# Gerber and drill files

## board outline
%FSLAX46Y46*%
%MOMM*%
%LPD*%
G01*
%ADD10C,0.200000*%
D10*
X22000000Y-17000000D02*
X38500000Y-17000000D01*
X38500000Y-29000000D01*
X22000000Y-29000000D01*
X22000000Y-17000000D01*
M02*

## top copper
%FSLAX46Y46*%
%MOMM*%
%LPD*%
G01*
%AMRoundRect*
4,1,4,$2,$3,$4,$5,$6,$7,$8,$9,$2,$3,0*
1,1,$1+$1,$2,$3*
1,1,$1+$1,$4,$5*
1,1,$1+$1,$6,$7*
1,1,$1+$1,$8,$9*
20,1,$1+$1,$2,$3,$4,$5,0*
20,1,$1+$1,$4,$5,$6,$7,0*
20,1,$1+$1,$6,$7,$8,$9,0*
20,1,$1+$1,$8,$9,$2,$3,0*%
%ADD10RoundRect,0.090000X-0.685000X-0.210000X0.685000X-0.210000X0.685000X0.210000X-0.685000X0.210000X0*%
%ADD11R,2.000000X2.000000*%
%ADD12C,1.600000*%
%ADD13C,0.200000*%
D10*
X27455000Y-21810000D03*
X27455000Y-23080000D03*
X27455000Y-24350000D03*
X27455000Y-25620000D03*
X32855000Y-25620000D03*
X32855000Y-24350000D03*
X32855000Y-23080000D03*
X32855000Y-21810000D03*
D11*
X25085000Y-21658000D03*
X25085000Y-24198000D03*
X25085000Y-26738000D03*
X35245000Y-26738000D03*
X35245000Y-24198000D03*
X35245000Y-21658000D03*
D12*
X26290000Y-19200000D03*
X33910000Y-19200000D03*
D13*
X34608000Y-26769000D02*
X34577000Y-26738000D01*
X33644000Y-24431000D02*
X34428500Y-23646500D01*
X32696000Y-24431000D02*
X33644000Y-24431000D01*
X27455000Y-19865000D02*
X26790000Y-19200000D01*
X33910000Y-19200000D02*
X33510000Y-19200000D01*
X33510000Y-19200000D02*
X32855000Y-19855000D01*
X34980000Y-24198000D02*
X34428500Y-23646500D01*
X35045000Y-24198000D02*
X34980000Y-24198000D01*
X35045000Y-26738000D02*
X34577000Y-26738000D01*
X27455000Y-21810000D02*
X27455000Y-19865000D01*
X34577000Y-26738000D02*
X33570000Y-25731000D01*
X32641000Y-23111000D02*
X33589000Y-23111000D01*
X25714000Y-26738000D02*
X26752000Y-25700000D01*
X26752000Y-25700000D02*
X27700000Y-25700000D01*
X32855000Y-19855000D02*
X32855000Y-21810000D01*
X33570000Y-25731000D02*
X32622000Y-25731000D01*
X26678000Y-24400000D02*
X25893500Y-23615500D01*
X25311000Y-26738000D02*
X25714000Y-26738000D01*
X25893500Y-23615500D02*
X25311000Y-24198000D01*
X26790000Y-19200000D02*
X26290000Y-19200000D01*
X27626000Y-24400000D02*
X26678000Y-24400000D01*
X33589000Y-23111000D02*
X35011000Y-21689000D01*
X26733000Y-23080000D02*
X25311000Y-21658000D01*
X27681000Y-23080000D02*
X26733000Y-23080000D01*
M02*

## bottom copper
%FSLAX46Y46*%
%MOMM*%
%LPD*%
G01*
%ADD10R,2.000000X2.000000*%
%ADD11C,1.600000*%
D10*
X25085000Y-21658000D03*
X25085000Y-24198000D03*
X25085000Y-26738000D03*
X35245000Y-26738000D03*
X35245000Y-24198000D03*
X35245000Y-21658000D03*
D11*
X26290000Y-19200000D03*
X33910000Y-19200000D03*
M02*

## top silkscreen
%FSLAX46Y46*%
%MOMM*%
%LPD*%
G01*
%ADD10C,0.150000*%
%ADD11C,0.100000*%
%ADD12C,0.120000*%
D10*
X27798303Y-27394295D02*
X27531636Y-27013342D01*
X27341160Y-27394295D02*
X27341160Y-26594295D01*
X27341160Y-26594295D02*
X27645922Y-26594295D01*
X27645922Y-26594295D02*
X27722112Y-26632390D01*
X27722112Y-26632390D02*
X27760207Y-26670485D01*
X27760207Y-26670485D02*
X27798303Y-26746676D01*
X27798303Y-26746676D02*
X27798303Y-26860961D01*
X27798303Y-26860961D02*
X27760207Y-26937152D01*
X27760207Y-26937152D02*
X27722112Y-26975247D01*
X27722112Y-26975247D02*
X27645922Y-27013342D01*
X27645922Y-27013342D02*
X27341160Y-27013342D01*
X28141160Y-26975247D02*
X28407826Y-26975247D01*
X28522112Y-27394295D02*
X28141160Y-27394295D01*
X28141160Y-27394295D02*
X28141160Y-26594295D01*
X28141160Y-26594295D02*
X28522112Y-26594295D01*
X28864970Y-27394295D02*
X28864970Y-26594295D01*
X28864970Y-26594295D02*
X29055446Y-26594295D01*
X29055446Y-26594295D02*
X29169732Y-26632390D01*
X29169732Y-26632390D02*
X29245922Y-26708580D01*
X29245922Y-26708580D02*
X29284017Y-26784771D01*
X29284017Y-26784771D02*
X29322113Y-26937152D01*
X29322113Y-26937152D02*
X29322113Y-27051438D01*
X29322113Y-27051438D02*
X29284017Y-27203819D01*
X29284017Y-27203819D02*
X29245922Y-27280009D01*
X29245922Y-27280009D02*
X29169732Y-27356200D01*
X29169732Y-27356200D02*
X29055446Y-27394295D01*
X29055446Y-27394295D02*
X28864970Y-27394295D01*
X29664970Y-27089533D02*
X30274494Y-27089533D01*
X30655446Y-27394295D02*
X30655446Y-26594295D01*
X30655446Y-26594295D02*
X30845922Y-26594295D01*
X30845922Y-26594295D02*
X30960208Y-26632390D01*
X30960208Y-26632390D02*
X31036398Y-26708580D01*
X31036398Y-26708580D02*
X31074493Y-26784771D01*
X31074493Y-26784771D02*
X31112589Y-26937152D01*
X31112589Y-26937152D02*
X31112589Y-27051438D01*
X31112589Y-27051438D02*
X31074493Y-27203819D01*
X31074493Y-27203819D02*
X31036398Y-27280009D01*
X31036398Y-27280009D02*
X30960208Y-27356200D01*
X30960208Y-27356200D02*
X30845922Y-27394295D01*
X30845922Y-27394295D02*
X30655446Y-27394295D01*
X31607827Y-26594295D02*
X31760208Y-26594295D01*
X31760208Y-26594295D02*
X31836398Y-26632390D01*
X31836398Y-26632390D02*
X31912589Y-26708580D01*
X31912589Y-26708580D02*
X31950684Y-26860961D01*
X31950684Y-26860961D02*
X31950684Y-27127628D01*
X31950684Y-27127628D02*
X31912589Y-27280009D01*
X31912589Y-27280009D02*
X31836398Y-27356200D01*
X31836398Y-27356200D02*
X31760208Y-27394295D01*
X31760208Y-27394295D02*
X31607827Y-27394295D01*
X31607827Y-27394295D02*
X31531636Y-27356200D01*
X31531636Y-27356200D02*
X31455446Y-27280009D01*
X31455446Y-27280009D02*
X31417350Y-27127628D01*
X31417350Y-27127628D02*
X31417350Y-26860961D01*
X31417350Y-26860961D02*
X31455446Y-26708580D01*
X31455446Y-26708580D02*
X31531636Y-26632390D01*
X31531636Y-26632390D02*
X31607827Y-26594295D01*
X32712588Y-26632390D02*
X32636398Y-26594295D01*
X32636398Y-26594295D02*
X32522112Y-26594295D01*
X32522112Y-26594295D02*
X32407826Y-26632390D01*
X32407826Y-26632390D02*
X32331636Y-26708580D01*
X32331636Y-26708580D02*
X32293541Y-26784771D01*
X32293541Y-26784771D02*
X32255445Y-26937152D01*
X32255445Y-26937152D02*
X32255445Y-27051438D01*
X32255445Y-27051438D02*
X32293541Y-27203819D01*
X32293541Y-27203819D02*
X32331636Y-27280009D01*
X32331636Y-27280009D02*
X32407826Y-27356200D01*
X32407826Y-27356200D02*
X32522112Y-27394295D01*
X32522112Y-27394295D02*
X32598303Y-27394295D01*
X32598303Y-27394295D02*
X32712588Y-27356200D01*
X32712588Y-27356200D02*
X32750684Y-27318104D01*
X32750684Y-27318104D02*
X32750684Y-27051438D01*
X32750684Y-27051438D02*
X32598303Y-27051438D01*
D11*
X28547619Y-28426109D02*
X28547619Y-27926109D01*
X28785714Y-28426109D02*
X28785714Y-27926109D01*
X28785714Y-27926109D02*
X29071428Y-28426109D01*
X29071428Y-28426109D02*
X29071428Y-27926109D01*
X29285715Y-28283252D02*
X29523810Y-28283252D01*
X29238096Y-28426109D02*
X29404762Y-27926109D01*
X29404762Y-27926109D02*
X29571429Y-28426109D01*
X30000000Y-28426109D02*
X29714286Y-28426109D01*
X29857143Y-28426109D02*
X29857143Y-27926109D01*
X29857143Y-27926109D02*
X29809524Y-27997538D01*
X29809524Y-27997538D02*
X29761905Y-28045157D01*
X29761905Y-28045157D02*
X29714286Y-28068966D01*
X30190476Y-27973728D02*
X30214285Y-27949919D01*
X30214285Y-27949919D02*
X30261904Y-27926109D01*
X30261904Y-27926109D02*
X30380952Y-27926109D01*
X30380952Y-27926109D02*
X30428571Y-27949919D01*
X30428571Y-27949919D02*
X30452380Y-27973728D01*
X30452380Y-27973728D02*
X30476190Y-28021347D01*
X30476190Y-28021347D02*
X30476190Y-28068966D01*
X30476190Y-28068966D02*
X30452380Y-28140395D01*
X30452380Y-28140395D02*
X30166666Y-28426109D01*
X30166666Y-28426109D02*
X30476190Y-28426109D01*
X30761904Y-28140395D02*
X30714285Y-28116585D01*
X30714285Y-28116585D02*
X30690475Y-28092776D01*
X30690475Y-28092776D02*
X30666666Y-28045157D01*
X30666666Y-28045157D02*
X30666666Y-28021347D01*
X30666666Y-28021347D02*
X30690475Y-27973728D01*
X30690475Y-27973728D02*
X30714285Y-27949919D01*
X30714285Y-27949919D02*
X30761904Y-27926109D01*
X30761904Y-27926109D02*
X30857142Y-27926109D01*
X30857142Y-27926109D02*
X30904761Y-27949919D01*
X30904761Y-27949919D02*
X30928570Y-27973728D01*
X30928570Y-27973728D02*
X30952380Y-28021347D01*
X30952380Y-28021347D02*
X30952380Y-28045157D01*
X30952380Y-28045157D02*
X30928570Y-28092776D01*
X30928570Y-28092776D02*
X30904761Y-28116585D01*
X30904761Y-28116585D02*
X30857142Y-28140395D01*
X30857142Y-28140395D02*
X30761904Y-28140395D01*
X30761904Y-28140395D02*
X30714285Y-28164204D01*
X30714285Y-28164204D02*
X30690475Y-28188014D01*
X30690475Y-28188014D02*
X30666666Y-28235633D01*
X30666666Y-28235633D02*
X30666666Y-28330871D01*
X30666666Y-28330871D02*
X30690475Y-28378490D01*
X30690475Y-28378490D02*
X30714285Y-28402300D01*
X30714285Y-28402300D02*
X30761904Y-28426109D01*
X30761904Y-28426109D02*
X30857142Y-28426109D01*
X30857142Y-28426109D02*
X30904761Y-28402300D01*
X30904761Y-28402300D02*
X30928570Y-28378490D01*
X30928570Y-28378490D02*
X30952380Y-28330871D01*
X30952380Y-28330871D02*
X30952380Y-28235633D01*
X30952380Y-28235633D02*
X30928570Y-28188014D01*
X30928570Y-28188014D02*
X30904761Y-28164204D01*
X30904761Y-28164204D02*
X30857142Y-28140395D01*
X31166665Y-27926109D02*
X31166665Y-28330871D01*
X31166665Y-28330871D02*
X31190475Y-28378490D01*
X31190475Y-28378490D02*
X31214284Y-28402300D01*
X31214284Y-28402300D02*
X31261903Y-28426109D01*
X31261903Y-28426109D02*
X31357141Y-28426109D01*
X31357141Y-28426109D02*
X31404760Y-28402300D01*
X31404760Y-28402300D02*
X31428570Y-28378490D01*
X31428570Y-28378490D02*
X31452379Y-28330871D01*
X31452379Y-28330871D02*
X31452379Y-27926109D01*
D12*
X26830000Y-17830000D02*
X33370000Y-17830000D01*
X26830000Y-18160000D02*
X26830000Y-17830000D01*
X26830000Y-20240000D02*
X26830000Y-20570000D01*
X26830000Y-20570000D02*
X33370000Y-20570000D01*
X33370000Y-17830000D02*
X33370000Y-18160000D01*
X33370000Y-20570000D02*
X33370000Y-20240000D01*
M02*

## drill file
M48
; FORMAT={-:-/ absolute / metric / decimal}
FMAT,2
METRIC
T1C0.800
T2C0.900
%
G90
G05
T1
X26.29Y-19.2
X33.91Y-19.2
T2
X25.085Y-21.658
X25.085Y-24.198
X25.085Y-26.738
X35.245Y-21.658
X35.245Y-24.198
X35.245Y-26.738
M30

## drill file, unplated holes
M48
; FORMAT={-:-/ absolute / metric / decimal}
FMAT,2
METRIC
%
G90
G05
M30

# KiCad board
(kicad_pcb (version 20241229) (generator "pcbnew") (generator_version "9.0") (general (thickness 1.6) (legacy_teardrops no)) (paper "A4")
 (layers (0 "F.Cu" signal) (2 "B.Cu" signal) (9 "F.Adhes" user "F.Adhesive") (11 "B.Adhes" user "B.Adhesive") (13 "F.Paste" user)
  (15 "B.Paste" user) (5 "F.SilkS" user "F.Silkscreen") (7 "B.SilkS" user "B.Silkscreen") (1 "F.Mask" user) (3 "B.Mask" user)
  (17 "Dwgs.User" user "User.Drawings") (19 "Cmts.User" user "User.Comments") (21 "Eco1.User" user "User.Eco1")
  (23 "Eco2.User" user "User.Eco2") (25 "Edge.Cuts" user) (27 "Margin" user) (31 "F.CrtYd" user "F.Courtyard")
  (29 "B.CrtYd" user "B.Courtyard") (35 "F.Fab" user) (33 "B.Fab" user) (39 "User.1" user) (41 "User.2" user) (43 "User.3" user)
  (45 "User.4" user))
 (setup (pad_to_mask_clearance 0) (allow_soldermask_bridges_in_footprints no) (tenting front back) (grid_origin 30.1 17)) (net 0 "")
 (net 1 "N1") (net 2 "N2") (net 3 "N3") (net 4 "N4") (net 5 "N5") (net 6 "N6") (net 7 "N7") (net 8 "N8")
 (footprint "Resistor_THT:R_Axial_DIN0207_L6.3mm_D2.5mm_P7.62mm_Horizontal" (layer "F.Cu") (at 26.29 19.2)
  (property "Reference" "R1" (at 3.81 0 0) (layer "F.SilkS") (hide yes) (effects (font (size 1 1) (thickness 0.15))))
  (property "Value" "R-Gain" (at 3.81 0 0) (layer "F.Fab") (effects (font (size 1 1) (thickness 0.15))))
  (fp_line (start 0.54 -1.37) (end 7.08 -1.37) (stroke (width 0.12) (type solid)) (layer "F.SilkS"))
  (fp_line (start 0.54 -1.04) (end 0.54 -1.37) (stroke (width 0.12) (type solid)) (layer "F.SilkS"))
  (fp_line (start 0.54 1.04) (end 0.54 1.37) (stroke (width 0.12) (type solid)) (layer "F.SilkS"))
  (fp_line (start 0.54 1.37) (end 7.08 1.37) (stroke (width 0.12) (type solid)) (layer "F.SilkS"))
  (fp_line (start 7.08 -1.37) (end 7.08 -1.04) (stroke (width 0.12) (type solid)) (layer "F.SilkS"))
  (fp_line (start 7.08 1.37) (end 7.08 1.04) (stroke (width 0.12) (type solid)) (layer "F.SilkS"))
  (pad "1" thru_hole circle (at 0 0) (size 1.6 1.6) (drill 0.8) (layers "*.Cu" "*.Mask") (remove_unused_layers no) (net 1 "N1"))
  (pad "2" thru_hole circle (at 7.62 0) (size 1.6 1.6) (drill 0.8) (layers "*.Cu" "*.Mask") (remove_unused_layers no) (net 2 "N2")))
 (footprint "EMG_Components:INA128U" (layer "F.Cu") (at 30.19 24.198)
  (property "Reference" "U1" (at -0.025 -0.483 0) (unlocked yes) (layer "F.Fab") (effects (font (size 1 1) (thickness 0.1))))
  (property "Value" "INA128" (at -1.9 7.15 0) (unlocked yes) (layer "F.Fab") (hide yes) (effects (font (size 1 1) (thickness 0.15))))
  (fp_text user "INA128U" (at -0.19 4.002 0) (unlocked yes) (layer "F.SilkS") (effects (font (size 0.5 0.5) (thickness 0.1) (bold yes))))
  (pad "1" smd roundrect (at -2.735 -2.388) (size 1.55 0.6) (layers "F.Cu" "F.Mask" "F.Paste") (roundrect_rratio 0.15) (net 1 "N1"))
  (pad "2" smd roundrect (at -2.735 -1.118) (size 1.55 0.6) (layers "F.Cu" "F.Mask" "F.Paste") (roundrect_rratio 0.15) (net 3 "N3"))
  (pad "3" smd roundrect (at -2.735 0.152) (size 1.55 0.6) (layers "F.Cu" "F.Mask" "F.Paste") (roundrect_rratio 0.15) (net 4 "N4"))
  (pad "4" smd roundrect (at -2.735 1.422) (size 1.55 0.6) (layers "F.Cu" "F.Mask" "F.Paste") (roundrect_rratio 0.15) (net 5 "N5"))
  (pad "5" smd roundrect (at 2.665 1.422) (size 1.55 0.6) (layers "F.Cu" "F.Mask" "F.Paste") (roundrect_rratio 0.15) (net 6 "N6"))
  (pad "6" smd roundrect (at 2.665 0.152) (size 1.55 0.6) (layers "F.Cu" "F.Mask" "F.Paste") (roundrect_rratio 0.15) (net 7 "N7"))
  (pad "7" smd roundrect (at 2.665 -1.118) (size 1.55 0.6) (layers "F.Cu" "F.Mask" "F.Paste") (roundrect_rratio 0.15) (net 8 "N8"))
  (pad "8" smd roundrect (at 2.665 -2.388) (size 1.55 0.6) (layers "F.Cu" "F.Mask" "F.Paste") (roundrect_rratio 0.15) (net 2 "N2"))
  (pad "T2" thru_hole rect (at -5.105 -2.54 180) (size 2 2) (drill 0.9) (layers "*.Cu" "*.Mask") (remove_unused_layers no) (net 3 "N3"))
  (pad "T3" thru_hole rect (at -5.105 0 180) (size 2 2) (drill 0.9) (layers "*.Cu" "*.Mask") (remove_unused_layers no) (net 4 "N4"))
  (pad "T4" thru_hole rect (at -5.105 2.54 180) (size 2 2) (drill 0.9) (layers "*.Cu" "*.Mask") (remove_unused_layers no) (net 5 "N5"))
  (pad "T5" thru_hole rect (at 5.055 2.54 180) (size 2 2) (drill 0.9) (layers "*.Cu" "*.Mask") (remove_unused_layers no) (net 6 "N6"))
  (pad "T6" thru_hole rect (at 5.055 0 180) (size 2 2) (drill 0.9) (layers "*.Cu" "*.Mask") (remove_unused_layers no) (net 7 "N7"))
  (pad "T7" thru_hole rect (at 5.055 -2.54 180) (size 2 2) (drill 0.9) (layers "*.Cu" "*.Mask") (remove_unused_layers no) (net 8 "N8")))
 (gr_rect (start 22 17) (end 38.5 29) (stroke (width 0.2) (type solid)) (fill no) (layer "Edge.Cuts"))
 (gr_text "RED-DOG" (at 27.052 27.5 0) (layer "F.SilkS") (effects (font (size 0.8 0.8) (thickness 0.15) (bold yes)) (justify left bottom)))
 (segment (start 27.626 24.4) (end 26.678 24.4) (width 0.2) (layer "F.Cu") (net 4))
 (segment (start 26.678 24.4) (end 25.8935 23.6155) (width 0.2) (layer "F.Cu") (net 4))
 (segment (start 25.8935 23.6155) (end 25.311 24.198) (width 0.2) (layer "F.Cu") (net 4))
 (segment (start 25.714 26.738) (end 26.752 25.7) (width 0.2) (layer "F.Cu") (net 5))
 (segment (start 26.752 25.7) (end 27.7 25.7) (width 0.2) (layer "F.Cu") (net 5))
 (segment (start 25.311 26.738) (end 25.714 26.738) (width 0.2) (layer "F.Cu") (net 5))
 (segment (start 27.455 21.81) (end 27.455 19.865) (width 0.2) (layer "F.Cu") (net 1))
 (segment (start 26.79 19.2) (end 26.29 19.2) (width 0.2) (layer "F.Cu") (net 1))
 (segment (start 27.455 19.865) (end 26.79 19.2) (width 0.2) (layer "F.Cu") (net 1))
 (segment (start 33.644 24.431) (end 34.4285 23.6465) (width 0.2) (layer "F.Cu") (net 7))
 (segment (start 35.045 24.198) (end 34.98 24.198) (width 0.2) (layer "F.Cu") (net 7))
 (segment (start 34.98 24.198) (end 34.4285 23.6465) (width 0.2) (layer "F.Cu") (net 7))
 (segment (start 32.696 24.431) (end 33.644 24.431) (width 0.2) (layer "F.Cu") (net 7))
 (segment (start 26.733 23.08) (end 25.311 21.658) (width 0.2) (layer "F.Cu") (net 3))
 (segment (start 27.681 23.08) (end 26.733 23.08) (width 0.2) (layer "F.Cu") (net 3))
 (segment (start 33.589 23.111) (end 35.011 21.689) (width 0.2) (layer "F.Cu") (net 8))
 (segment (start 32.641 23.111) (end 33.589 23.111) (width 0.2) (layer "F.Cu") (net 8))
 (segment (start 35.045 26.738) (end 34.577 26.738) (width 0.2) (layer "F.Cu") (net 6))
 (segment (start 33.57 25.731) (end 32.622 25.731) (width 0.2) (layer "F.Cu") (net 6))
 (segment (start 34.577 26.738) (end 33.57 25.731) (width 0.2) (layer "F.Cu") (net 6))
 (segment (start 34.608 26.769) (end 34.577 26.738) (width 0.2) (layer "F.Cu") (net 6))
 (segment (start 32.855 19.855) (end 32.855 21.81) (width 0.2) (layer "F.Cu") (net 2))
 (segment (start 33.51 19.2) (end 32.855 19.855) (width 0.2) (layer "F.Cu") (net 2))
 (segment (start 33.91 19.2) (end 33.51 19.2) (width 0.2) (layer "F.Cu") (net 2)))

